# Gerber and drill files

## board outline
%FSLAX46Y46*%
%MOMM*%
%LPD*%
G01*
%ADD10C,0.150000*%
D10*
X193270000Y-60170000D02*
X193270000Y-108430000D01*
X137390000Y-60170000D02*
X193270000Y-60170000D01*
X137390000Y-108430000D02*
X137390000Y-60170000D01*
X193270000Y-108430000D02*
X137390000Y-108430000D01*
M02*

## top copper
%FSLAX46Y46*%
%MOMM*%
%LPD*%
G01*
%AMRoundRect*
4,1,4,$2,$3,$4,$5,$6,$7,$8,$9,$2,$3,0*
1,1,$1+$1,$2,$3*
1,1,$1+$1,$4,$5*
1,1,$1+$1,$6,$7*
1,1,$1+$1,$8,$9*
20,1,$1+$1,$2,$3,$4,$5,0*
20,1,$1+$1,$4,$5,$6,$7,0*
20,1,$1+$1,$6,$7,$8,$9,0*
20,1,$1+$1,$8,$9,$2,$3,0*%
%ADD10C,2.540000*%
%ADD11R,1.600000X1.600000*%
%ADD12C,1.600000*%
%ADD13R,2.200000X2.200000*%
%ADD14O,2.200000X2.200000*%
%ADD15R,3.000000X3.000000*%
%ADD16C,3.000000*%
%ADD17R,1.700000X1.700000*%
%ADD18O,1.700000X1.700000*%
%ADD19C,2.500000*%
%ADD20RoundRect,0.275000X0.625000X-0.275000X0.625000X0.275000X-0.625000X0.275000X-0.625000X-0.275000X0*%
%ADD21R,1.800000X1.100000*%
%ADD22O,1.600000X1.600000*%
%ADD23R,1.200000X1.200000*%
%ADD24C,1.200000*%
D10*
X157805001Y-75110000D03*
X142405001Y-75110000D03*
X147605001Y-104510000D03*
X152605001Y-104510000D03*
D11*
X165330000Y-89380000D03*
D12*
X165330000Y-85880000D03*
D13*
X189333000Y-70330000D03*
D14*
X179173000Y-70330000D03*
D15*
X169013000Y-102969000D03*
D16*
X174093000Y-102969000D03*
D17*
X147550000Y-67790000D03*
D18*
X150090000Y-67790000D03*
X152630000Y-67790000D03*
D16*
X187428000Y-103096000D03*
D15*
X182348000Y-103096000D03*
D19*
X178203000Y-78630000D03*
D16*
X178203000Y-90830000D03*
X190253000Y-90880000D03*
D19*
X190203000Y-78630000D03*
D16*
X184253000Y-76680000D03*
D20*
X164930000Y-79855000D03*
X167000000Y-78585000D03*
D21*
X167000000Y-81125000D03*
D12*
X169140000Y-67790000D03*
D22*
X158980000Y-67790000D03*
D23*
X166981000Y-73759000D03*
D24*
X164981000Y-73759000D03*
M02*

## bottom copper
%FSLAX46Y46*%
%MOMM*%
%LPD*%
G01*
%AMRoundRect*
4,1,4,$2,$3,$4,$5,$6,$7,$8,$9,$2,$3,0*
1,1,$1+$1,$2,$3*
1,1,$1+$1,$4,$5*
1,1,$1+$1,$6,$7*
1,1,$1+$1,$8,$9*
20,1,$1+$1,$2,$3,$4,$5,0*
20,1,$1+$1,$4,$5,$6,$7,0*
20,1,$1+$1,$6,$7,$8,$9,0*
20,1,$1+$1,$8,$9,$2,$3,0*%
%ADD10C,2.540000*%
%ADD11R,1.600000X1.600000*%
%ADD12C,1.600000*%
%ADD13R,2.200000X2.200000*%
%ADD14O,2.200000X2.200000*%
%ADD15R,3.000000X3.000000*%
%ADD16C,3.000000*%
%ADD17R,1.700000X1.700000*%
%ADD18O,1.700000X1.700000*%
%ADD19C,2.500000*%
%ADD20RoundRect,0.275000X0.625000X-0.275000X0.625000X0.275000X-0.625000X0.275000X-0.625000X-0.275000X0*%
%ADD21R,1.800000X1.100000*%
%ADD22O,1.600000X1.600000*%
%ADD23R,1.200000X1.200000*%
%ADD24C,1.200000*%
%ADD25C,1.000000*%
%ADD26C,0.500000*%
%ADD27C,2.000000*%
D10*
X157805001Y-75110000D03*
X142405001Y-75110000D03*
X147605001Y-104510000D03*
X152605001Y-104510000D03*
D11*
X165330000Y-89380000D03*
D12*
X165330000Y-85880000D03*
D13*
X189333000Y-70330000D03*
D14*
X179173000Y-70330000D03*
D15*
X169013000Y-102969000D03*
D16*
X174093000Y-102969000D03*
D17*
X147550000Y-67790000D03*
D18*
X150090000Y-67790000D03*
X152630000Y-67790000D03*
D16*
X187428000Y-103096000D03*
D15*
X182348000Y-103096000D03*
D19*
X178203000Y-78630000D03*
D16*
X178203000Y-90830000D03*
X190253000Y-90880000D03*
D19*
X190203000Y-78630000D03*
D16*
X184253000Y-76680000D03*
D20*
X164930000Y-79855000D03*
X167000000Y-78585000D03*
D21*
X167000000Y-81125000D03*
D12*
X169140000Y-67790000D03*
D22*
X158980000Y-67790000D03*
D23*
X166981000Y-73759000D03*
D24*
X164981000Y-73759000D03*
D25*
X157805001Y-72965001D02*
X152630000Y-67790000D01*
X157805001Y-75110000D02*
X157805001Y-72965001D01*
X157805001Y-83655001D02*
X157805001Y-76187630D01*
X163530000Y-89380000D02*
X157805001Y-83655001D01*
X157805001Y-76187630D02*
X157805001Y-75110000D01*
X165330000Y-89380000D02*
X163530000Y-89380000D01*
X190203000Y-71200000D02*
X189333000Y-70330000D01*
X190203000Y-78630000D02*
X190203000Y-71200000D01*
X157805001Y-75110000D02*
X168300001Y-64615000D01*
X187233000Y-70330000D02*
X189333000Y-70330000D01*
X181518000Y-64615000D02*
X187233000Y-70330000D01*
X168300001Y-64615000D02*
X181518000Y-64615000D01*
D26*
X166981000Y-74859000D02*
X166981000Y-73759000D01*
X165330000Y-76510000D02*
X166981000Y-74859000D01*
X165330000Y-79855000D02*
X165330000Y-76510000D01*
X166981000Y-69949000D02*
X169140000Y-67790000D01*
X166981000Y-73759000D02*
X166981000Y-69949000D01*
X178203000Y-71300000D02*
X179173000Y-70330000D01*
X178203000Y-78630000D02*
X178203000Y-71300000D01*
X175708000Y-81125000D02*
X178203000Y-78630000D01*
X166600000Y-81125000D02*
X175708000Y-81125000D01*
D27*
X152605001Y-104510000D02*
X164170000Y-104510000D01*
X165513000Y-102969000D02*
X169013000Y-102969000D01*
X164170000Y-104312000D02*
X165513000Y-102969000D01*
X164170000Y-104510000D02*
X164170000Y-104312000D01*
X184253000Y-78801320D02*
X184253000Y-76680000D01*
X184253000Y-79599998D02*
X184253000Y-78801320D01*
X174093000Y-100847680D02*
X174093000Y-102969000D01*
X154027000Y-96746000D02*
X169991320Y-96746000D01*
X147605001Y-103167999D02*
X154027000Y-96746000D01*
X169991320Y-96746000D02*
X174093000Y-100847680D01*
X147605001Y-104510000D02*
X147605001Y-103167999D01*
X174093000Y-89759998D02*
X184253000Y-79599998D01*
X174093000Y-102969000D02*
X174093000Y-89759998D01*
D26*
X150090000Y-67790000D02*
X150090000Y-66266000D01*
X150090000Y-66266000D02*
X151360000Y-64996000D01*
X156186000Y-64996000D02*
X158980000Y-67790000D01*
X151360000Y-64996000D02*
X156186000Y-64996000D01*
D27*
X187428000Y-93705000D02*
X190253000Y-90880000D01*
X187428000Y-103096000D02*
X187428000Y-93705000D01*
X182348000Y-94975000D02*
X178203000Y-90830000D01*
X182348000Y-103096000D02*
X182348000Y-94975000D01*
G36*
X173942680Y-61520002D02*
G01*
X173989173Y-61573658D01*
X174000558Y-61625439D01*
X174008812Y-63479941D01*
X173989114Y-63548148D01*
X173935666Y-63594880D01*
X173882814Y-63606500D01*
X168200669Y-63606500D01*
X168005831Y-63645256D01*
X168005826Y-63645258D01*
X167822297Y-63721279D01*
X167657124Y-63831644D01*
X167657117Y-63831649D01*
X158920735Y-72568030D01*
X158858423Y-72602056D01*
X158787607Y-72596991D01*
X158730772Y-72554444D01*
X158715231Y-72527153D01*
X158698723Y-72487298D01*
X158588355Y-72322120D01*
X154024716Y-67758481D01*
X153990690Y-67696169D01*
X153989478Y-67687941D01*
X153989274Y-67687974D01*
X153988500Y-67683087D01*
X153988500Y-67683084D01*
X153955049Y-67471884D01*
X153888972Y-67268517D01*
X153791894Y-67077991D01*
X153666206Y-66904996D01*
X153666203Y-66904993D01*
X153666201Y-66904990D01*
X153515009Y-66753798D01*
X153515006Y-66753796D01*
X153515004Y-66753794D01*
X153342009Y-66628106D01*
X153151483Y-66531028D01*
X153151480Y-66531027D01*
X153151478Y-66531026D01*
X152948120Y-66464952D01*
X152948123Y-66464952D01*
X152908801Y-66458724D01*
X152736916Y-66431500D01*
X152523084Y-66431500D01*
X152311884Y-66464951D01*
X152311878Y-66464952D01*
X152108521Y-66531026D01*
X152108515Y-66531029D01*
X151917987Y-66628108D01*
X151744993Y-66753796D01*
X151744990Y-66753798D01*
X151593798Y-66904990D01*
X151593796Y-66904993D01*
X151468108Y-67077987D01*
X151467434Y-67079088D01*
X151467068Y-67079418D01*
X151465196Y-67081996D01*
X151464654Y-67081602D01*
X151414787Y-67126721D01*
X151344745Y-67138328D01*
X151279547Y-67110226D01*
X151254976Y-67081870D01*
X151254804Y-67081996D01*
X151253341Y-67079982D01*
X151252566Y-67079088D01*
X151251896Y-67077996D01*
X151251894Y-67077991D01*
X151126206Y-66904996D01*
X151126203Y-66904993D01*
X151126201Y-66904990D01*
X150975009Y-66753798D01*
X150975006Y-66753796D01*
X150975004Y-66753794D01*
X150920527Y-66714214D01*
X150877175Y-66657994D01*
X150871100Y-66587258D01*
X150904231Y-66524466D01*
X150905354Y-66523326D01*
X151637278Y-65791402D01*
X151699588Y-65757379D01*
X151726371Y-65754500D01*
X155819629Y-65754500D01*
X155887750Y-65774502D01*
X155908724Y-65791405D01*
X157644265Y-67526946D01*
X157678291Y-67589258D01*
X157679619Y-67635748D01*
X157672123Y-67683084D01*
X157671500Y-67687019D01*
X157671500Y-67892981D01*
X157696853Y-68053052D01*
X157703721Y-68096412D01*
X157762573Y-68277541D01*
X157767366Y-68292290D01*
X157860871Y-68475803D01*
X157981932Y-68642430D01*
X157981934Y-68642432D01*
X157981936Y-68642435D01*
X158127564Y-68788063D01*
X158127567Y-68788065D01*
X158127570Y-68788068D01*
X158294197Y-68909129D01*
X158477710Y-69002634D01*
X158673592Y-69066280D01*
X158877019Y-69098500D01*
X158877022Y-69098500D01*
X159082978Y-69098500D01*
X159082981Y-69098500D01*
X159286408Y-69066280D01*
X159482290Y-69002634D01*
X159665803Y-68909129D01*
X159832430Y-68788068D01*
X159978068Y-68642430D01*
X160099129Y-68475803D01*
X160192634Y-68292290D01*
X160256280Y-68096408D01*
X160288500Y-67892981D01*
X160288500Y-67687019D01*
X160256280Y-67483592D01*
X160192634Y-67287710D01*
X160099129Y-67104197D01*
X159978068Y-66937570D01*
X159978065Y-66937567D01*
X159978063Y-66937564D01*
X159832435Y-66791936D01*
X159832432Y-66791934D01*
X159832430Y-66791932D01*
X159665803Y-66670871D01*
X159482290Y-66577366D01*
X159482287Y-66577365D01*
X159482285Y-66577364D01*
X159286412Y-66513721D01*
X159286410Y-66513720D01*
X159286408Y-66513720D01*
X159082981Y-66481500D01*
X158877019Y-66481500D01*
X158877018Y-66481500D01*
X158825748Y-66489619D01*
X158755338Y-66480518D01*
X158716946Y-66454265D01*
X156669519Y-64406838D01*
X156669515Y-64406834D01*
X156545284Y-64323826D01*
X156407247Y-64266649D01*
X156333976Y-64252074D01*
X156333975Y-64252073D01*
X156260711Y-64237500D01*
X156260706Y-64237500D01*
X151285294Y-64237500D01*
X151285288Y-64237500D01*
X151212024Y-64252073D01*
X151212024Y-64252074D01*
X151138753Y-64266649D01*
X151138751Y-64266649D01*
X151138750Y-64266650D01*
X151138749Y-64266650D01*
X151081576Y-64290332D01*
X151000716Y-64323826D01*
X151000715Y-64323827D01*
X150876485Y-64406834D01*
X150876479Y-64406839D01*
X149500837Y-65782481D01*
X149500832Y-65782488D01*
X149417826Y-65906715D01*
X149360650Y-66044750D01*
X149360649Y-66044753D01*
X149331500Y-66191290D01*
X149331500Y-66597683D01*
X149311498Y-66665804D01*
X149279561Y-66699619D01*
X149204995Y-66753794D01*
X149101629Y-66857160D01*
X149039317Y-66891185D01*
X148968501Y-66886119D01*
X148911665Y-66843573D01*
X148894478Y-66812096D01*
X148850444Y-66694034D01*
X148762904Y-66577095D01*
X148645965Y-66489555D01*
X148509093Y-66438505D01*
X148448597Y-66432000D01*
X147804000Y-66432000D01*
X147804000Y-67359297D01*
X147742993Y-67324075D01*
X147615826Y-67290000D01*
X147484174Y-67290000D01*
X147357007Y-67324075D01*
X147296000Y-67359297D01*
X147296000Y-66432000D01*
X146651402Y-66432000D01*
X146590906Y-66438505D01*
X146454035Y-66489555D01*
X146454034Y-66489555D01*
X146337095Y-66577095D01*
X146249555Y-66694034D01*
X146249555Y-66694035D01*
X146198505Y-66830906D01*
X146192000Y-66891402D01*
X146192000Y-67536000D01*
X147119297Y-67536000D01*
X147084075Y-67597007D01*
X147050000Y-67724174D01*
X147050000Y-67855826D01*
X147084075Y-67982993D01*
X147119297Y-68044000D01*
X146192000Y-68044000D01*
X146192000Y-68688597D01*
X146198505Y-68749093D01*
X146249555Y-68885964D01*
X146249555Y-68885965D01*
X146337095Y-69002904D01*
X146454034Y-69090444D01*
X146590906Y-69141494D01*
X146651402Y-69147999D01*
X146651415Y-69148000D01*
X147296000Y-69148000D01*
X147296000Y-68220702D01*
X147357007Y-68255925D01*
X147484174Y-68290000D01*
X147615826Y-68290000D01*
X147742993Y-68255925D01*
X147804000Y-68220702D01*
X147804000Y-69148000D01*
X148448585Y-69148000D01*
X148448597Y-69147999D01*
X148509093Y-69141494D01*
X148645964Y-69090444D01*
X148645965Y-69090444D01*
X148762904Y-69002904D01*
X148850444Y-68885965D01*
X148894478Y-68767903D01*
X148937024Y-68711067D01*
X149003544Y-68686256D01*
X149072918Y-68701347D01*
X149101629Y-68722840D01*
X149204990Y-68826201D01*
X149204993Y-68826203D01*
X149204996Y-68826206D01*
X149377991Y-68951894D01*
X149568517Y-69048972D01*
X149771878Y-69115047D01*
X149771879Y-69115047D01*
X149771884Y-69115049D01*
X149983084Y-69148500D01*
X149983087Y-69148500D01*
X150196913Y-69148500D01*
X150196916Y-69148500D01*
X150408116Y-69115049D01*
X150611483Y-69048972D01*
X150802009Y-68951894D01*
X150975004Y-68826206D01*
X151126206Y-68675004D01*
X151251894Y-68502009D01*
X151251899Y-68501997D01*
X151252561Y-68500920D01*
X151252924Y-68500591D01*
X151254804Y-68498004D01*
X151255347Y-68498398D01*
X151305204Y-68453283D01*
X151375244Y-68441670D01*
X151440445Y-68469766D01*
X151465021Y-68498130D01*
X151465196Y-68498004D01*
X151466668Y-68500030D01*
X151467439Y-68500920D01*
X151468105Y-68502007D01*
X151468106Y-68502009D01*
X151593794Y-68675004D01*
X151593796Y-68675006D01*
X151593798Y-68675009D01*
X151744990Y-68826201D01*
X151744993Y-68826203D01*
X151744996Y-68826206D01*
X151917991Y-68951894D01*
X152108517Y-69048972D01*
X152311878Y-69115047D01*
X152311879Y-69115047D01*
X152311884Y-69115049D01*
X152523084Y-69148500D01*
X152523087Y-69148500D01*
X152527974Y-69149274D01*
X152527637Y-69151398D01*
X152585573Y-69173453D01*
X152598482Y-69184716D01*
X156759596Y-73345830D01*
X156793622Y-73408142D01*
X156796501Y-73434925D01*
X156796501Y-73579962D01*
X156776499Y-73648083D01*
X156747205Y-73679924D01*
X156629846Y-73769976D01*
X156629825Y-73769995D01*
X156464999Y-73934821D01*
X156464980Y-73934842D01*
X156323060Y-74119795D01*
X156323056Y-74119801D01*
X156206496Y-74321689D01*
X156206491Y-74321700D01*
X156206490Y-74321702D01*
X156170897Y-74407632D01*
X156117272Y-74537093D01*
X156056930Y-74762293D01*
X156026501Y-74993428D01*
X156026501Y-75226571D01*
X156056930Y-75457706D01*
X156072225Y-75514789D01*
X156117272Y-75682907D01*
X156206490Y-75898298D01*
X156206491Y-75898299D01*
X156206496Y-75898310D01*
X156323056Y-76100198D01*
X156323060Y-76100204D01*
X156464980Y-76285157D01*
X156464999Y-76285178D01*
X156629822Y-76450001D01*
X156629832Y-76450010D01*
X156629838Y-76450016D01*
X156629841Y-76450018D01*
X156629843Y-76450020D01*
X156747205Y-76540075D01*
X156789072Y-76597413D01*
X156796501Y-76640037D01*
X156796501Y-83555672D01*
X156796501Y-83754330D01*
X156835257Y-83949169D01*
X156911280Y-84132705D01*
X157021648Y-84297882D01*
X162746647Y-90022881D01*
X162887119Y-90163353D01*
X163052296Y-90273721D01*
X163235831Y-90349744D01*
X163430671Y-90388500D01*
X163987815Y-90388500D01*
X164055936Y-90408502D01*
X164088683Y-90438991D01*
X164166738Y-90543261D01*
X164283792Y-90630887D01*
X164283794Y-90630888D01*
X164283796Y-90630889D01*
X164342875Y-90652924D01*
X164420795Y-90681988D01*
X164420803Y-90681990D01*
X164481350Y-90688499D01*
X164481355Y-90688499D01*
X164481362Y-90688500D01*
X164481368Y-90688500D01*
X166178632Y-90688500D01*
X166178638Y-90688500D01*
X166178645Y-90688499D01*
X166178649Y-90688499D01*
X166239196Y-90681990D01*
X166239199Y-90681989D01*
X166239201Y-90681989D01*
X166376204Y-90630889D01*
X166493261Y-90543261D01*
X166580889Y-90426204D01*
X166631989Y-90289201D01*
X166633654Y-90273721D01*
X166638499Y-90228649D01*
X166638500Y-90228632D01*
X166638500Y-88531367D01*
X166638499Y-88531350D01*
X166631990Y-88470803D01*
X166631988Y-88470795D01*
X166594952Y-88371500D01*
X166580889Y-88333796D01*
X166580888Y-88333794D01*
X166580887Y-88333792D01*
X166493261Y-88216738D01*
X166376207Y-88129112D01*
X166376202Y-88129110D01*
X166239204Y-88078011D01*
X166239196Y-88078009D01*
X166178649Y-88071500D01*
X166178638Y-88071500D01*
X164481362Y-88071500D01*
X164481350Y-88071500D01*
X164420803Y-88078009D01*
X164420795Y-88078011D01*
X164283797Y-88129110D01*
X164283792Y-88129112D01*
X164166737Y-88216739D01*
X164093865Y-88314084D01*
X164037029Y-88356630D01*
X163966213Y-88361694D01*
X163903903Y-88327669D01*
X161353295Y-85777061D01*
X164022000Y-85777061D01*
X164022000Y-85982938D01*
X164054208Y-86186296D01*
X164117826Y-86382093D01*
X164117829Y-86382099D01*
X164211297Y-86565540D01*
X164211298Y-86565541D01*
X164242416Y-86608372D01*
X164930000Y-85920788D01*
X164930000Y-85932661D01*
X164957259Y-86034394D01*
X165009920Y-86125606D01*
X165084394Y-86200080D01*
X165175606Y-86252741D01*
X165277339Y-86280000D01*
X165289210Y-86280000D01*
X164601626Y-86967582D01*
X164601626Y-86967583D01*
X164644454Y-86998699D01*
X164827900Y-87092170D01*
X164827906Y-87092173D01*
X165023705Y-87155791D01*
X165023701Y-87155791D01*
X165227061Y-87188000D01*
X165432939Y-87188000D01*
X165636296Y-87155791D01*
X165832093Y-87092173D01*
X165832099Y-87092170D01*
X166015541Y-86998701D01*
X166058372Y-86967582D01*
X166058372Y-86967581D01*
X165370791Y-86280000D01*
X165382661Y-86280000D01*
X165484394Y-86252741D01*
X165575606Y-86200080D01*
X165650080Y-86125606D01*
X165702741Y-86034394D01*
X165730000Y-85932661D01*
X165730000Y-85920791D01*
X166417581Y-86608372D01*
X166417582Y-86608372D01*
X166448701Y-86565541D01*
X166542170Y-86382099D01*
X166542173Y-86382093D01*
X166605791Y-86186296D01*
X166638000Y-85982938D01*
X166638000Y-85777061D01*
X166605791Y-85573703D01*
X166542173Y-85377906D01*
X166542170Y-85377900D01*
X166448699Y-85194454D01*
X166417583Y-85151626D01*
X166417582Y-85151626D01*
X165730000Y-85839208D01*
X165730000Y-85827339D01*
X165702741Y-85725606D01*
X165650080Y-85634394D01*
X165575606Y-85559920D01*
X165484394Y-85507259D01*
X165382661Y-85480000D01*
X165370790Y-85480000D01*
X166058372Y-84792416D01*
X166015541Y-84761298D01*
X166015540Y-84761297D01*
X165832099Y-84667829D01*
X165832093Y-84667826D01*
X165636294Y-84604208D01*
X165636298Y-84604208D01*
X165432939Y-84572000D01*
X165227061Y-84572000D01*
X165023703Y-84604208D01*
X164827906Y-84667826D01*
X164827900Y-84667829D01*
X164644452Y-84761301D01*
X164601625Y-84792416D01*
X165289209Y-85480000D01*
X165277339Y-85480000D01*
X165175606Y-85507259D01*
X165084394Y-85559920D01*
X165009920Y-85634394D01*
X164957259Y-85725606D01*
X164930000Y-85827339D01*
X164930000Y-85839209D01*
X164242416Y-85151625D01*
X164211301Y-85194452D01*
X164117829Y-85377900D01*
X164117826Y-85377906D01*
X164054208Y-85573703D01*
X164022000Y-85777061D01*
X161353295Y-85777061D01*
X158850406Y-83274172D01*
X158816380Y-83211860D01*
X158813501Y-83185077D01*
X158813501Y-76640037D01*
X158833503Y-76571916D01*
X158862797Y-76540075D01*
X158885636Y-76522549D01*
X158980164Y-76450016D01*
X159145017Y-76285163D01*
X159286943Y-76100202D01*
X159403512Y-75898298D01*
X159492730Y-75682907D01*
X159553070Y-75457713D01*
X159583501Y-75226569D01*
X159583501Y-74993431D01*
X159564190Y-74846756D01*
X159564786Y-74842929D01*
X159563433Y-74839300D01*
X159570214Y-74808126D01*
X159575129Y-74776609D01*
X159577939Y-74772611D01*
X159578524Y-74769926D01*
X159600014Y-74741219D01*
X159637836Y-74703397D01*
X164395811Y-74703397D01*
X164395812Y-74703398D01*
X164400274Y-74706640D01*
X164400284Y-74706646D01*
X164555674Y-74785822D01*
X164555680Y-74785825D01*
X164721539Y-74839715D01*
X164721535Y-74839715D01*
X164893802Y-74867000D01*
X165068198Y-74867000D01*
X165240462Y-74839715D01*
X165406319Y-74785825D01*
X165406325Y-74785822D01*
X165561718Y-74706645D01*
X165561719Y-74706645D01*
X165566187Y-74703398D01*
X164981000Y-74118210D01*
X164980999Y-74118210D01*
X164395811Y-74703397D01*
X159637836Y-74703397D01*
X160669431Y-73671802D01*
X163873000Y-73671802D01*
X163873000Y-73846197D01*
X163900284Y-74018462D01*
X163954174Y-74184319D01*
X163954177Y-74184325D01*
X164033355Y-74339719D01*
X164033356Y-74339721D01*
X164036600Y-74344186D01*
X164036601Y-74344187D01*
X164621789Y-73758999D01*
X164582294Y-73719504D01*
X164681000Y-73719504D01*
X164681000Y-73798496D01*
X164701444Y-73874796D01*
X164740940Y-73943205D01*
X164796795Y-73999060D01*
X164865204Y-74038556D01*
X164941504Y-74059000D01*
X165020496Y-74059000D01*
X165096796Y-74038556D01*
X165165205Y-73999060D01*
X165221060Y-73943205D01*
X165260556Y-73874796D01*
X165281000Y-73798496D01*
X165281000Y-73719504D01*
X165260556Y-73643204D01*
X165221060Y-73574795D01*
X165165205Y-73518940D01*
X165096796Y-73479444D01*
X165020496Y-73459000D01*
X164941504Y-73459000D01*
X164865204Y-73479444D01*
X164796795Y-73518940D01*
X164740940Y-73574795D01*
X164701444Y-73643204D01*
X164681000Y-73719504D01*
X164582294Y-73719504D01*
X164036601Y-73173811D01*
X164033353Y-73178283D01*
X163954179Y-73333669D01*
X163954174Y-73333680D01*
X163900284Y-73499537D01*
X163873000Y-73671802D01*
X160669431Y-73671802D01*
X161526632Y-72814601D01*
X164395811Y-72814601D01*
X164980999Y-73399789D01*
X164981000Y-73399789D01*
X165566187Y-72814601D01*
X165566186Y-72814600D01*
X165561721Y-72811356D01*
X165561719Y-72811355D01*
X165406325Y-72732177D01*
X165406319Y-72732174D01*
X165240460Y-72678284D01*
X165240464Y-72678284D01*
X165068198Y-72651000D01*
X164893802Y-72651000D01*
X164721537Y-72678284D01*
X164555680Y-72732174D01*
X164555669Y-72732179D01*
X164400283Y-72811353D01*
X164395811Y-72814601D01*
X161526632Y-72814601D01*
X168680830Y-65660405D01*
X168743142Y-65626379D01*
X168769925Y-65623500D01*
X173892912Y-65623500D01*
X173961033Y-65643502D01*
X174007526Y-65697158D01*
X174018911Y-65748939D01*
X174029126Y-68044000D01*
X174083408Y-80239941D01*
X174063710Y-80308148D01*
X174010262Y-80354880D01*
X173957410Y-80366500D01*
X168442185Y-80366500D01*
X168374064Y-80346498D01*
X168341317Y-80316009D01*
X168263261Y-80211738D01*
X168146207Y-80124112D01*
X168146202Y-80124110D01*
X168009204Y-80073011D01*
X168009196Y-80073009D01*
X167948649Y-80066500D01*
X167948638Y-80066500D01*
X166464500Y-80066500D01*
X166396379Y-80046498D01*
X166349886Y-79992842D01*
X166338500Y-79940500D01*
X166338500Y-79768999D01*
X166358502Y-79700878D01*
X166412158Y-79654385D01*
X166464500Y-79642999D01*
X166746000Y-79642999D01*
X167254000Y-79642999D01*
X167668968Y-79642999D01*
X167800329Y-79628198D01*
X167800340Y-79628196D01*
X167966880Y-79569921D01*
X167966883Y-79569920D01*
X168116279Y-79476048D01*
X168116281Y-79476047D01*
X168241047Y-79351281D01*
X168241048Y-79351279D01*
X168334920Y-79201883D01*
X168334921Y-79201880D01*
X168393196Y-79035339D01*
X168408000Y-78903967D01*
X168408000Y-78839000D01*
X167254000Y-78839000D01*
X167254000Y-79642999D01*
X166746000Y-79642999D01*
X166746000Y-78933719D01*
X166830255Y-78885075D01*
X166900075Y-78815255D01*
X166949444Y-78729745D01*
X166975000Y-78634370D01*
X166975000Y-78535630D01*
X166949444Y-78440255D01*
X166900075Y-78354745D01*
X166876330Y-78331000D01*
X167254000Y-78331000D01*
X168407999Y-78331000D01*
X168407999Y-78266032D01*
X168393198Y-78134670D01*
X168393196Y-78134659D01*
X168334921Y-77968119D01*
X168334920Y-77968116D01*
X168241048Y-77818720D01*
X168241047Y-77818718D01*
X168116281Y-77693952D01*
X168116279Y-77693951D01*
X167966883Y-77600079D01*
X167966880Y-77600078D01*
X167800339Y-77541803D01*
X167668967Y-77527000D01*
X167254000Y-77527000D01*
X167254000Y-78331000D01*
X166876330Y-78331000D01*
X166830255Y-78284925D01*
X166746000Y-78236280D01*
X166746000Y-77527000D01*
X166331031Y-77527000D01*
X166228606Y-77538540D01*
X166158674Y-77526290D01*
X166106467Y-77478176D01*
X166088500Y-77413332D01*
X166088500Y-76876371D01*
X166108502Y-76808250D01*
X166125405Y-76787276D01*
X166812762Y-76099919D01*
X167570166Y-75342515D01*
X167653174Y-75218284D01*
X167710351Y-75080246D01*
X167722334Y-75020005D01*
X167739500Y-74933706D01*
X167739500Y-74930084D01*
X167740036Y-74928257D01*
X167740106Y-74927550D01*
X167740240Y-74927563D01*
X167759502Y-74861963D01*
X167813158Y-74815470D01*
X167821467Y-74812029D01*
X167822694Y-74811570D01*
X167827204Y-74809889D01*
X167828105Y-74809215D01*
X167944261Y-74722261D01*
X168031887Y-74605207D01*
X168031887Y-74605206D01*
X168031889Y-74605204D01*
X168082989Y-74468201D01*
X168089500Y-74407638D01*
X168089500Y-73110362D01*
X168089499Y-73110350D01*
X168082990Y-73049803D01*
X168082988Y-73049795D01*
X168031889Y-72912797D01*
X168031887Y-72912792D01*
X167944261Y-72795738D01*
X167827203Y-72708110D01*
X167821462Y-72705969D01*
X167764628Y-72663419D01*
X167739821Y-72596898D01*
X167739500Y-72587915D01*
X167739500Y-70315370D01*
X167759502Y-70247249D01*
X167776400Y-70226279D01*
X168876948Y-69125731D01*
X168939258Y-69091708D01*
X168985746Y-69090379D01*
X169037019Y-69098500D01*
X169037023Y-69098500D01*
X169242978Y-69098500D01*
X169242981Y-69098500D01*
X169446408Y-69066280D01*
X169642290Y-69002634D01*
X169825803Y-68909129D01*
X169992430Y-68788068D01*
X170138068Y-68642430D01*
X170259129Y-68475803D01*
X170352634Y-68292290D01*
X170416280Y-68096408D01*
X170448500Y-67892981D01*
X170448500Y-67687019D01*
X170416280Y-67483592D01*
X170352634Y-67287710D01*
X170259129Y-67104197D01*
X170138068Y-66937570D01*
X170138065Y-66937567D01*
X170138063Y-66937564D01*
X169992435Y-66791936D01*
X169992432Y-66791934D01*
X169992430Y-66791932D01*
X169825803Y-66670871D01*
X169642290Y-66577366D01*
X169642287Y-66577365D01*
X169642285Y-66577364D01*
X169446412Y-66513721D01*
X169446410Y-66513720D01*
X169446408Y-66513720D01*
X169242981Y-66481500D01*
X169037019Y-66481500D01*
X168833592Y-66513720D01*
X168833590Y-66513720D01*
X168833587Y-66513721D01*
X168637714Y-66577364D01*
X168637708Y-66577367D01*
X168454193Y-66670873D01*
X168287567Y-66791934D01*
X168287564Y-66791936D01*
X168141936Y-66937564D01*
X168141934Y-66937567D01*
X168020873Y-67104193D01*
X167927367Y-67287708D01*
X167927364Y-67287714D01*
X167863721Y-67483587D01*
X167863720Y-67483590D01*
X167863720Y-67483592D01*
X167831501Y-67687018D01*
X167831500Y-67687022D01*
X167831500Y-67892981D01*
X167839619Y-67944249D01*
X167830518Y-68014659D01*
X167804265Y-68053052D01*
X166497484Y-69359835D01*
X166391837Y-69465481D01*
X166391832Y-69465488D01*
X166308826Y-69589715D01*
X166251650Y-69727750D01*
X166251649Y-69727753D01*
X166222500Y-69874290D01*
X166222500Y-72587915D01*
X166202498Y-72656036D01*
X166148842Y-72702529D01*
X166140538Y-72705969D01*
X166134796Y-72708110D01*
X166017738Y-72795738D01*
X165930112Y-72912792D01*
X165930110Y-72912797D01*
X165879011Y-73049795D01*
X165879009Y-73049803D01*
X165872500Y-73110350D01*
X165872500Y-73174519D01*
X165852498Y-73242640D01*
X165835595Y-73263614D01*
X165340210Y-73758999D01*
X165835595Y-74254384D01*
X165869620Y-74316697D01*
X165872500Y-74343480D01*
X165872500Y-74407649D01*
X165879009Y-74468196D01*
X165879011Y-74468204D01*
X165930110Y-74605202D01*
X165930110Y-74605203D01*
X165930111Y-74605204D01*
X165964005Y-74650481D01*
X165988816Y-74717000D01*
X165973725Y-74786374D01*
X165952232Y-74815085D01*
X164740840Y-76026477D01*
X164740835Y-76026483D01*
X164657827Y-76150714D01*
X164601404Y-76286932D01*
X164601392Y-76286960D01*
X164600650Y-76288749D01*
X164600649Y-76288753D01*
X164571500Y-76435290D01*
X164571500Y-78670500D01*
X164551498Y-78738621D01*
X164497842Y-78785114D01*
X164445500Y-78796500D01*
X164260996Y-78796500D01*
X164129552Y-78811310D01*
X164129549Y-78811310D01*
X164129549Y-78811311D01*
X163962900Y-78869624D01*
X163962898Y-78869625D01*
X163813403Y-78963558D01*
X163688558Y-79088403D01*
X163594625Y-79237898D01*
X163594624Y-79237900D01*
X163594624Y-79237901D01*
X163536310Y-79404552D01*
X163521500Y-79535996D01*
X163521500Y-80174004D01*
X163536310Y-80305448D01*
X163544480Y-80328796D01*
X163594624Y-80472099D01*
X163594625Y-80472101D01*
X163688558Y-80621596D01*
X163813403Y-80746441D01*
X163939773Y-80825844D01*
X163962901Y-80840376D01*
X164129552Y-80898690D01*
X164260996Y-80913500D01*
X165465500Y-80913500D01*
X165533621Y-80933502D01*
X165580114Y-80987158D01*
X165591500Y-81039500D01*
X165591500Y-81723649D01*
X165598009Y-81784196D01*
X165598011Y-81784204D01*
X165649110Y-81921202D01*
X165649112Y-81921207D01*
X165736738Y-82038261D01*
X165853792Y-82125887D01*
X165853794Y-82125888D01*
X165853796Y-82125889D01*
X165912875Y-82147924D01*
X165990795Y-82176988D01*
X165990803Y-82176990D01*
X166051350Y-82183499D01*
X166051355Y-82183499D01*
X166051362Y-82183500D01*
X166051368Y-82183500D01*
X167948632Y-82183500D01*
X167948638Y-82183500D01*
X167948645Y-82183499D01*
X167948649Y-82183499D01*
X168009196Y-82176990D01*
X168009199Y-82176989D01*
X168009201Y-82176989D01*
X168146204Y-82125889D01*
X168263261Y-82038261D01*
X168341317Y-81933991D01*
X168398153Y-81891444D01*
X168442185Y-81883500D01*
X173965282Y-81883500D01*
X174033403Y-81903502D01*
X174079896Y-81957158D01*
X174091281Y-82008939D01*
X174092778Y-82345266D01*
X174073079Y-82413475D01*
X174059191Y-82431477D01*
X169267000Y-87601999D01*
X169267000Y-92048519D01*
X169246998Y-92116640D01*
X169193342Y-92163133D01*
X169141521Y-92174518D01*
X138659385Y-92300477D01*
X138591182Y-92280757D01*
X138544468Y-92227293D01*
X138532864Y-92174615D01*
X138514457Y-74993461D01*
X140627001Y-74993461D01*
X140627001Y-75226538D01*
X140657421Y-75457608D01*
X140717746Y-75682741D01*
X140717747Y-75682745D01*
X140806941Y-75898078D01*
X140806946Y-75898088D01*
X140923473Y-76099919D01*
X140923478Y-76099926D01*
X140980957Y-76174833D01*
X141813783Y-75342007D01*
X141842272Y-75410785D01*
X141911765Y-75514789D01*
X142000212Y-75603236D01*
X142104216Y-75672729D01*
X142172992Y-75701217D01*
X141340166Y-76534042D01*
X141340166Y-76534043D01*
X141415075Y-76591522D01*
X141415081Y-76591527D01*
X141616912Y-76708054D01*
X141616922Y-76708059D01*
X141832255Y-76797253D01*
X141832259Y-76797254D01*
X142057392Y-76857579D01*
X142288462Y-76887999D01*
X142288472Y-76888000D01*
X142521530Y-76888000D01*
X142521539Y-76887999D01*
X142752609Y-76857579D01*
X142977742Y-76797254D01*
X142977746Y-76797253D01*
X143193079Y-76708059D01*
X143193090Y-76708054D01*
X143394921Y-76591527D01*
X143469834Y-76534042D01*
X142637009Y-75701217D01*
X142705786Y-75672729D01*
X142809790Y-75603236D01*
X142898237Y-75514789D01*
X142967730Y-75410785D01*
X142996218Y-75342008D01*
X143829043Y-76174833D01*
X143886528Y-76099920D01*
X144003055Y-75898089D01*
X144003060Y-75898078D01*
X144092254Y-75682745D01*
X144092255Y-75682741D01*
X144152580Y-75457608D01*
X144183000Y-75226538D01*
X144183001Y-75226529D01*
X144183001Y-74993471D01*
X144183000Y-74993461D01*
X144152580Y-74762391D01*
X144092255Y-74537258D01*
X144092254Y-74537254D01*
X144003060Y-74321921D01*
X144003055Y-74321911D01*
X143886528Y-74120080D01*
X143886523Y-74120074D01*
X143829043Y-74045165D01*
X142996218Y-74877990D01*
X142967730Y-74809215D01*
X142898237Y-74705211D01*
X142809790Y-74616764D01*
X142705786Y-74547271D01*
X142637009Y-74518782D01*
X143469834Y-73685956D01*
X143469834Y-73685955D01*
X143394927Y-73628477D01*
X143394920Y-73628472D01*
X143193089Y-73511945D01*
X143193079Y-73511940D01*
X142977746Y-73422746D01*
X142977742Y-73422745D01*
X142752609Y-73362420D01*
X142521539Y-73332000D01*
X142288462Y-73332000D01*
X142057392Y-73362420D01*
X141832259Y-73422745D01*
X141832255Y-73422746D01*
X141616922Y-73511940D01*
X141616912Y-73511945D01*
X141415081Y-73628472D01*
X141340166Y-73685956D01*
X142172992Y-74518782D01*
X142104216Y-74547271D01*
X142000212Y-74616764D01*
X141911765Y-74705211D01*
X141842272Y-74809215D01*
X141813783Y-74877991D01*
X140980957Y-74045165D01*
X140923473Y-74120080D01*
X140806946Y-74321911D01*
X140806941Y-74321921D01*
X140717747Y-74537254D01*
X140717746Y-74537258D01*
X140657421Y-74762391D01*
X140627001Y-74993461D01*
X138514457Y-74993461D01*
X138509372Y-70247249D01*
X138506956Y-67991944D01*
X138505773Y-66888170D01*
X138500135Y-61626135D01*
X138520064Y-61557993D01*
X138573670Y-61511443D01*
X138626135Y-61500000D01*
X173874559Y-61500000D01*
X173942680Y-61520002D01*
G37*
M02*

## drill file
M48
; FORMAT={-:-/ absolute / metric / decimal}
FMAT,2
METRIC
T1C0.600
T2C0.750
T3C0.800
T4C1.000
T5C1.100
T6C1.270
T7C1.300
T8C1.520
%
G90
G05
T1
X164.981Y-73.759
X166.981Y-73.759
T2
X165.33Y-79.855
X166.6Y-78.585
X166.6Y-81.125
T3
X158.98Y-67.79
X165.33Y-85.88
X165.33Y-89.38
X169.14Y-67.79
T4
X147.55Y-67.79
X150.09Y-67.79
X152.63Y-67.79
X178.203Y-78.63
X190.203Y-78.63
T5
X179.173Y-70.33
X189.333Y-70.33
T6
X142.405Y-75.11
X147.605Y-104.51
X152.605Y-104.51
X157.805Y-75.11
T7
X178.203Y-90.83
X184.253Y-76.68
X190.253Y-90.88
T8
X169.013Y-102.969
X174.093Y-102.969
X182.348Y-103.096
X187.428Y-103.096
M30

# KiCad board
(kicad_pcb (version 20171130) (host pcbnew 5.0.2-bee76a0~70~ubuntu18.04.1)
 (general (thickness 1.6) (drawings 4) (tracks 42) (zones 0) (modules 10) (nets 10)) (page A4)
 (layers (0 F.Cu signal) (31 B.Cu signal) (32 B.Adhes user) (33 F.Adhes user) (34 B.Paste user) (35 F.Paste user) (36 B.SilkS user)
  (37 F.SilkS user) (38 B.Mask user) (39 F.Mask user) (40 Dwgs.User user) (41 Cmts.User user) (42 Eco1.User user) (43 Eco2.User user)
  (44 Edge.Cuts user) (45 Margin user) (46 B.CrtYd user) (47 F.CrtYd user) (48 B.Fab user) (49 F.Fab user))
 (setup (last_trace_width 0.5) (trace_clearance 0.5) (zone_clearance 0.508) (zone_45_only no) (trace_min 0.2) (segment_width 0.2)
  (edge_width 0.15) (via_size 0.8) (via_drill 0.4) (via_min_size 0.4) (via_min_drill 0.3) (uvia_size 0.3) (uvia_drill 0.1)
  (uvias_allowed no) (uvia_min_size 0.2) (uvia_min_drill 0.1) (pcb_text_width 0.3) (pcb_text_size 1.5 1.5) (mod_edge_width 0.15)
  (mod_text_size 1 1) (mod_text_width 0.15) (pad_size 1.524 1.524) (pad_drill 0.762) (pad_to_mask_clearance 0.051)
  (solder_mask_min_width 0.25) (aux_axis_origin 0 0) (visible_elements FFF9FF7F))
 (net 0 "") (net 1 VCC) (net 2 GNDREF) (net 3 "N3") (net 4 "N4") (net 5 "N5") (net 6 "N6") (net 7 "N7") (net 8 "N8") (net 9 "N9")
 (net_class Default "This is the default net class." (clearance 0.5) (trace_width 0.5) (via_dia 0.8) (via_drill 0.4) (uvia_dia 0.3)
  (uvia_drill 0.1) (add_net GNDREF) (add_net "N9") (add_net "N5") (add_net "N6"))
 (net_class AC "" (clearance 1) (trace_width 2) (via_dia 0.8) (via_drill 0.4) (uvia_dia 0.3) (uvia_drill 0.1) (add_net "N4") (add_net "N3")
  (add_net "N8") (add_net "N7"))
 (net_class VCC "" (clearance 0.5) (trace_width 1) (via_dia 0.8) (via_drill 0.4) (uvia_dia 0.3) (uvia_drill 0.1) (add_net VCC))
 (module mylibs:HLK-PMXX (layer F.Cu) (at 160.205001 106.91 90)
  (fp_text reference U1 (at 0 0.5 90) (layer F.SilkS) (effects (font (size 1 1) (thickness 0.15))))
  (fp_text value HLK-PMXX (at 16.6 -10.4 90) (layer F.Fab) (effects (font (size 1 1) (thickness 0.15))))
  (pad 4 thru_hole circle (at 31.8 -2.4 90) (size 2.54 2.54) (drill 1.27) (layers *.Cu *.Mask) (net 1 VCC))
  (pad 3 thru_hole circle (at 31.8 -17.8 90) (size 2.54 2.54) (drill 1.27) (layers *.Cu *.Mask) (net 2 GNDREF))
  (pad 1 thru_hole circle (at 2.4 -12.6 90) (size 2.54 2.54) (drill 1.27) (layers *.Cu *.Mask) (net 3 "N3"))
  (pad 2 thru_hole circle (at 2.4 -7.6 90) (size 2.54 2.54) (drill 1.27) (layers *.Cu *.Mask) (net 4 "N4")))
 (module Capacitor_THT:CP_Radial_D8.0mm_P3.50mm (layer F.Cu) (at 165.33 89.38 90)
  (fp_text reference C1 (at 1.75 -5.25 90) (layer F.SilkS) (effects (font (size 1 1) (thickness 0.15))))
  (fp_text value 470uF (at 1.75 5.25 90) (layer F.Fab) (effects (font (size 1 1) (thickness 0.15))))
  (pad 1 thru_hole rect (at 0 0 90) (size 1.6 1.6) (drill 0.8) (layers *.Cu *.Mask) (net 1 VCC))
  (pad 2 thru_hole circle (at 3.5 0 90) (size 1.6 1.6) (drill 0.8) (layers *.Cu *.Mask) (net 2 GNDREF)))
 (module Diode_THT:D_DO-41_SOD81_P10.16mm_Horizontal (layer F.Cu) (at 189.333 70.33 180)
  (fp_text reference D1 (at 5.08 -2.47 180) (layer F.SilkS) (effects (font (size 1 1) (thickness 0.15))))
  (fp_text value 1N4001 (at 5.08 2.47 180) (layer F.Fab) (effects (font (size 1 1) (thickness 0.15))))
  (pad 1 thru_hole rect (at 0 0 180) (size 2.2 2.2) (drill 1.1) (layers *.Cu *.Mask) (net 1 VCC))
  (pad 2 thru_hole oval (at 10.16 0 180) (size 2.2 2.2) (drill 1.1) (layers *.Cu *.Mask) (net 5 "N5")))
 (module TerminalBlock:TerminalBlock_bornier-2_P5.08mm (layer F.Cu) (at 169.013 102.969)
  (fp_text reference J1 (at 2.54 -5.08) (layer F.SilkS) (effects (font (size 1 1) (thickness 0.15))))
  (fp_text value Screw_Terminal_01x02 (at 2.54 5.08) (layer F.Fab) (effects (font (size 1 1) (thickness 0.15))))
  (pad 1 thru_hole rect (at 0 0) (size 3 3) (drill 1.52) (layers *.Cu *.Mask) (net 4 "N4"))
  (pad 2 thru_hole circle (at 5.08 0) (size 3 3) (drill 1.52) (layers *.Cu *.Mask) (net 3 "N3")))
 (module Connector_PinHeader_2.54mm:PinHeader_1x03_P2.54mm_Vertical (layer F.Cu) (at 147.55 67.79 90)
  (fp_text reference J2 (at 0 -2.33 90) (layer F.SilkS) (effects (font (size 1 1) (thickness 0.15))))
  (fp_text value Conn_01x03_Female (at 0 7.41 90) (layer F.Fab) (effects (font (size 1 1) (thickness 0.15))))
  (pad 1 thru_hole rect (at 0 0 90) (size 1.7 1.7) (drill 1) (layers *.Cu *.Mask) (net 2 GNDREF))
  (pad 2 thru_hole oval (at 0 2.54 90) (size 1.7 1.7) (drill 1) (layers *.Cu *.Mask) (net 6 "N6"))
  (pad 3 thru_hole oval (at 0 5.08 90) (size 1.7 1.7) (drill 1) (layers *.Cu *.Mask) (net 1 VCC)))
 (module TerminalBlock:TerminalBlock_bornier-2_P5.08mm (layer F.Cu) (at 182.348 103.096)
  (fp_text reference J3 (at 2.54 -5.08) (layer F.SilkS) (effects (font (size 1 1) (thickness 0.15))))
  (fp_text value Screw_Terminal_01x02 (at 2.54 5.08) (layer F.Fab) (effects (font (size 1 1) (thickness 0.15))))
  (pad 2 thru_hole circle (at 5.08 0) (size 3 3) (drill 1.52) (layers *.Cu *.Mask) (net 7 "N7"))
  (pad 1 thru_hole rect (at 0 0) (size 3 3) (drill 1.52) (layers *.Cu *.Mask) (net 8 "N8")))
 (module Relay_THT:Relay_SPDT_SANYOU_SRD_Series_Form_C (layer F.Cu) (at 184.253 76.68 270)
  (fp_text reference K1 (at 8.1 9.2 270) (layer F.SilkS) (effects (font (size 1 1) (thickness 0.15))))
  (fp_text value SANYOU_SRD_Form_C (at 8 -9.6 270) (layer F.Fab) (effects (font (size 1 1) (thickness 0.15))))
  (pad 2 thru_hole circle (at 1.95 6.05) (size 2.5 2.5) (drill 1) (layers *.Cu *.Mask) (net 5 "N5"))
  (pad 3 thru_hole circle (at 14.15 6.05) (size 3 3) (drill 1.3) (layers *.Cu *.Mask) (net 8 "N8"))
  (pad 4 thru_hole circle (at 14.2 -6) (size 3 3) (drill 1.3) (layers *.Cu *.Mask) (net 7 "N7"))
  (pad 5 thru_hole circle (at 1.95 -5.95) (size 2.5 2.5) (drill 1) (layers *.Cu *.Mask) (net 1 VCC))
  (pad 1 thru_hole circle (at 0 0) (size 3 3) (drill 1.3) (layers *.Cu *.Mask) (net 3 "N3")))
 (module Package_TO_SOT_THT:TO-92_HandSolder (layer F.Cu) (at 166.6 81.125 90)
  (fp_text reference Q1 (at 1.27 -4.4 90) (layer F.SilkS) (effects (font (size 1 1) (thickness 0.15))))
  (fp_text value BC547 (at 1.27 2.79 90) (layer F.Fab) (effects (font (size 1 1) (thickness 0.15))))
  (pad 2 thru_hole roundrect (at 1.27 -1.27 90) (size 1.1 1.8) (drill 0.75 (offset 0 -0.4)) (layers *.Cu *.Mask) (roundrect_rratio 0.25)
   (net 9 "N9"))
  (pad 3 thru_hole roundrect (at 2.54 0 90) (size 1.1 1.8) (drill 0.75 (offset 0 0.4)) (layers *.Cu *.Mask) (roundrect_rratio 0.25)
   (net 2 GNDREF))
  (pad 1 thru_hole rect (at 0 0 90) (size 1.1 1.8) (drill 0.75 (offset 0 0.4)) (layers *.Cu *.Mask) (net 5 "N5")))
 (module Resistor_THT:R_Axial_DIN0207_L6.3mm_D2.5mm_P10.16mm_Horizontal (layer F.Cu) (at 169.14 67.79 180)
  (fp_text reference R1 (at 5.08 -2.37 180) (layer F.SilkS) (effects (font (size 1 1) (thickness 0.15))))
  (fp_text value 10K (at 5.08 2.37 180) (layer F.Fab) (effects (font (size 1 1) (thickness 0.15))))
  (pad 1 thru_hole circle (at 0 0 180) (size 1.6 1.6) (drill 0.8) (layers *.Cu *.Mask) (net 9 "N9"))
  (pad 2 thru_hole oval (at 10.16 0 180) (size 1.6 1.6) (drill 0.8) (layers *.Cu *.Mask) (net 6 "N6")))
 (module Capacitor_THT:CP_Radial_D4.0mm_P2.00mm (layer F.Cu) (at 166.981 73.759 180)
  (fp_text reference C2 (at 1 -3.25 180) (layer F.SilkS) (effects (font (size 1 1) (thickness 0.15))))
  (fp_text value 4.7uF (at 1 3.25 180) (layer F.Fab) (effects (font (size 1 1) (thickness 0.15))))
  (pad 1 thru_hole rect (at 0 0 180) (size 1.2 1.2) (drill 0.6) (layers *.Cu *.Mask) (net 9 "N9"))
  (pad 2 thru_hole circle (at 2 0 180) (size 1.2 1.2) (drill 0.6) (layers *.Cu *.Mask) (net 2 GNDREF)))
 (gr_line (start 193.27 60.17) (end 193.27 108.43) (layer Edge.Cuts) (width 0.15))
 (gr_line (start 137.39 60.17) (end 193.27 60.17) (layer Edge.Cuts) (width 0.15))
 (gr_line (start 137.39 108.43) (end 137.39 60.17) (layer Edge.Cuts) (width 0.15))
 (gr_line (start 193.27 108.43) (end 137.39 108.43) (layer Edge.Cuts) (width 0.15))
 (segment (start 157.805001 72.965001) (end 152.63 67.79) (width 1) (layer B.Cu) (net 1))
 (segment (start 157.805001 75.11) (end 157.805001 72.965001) (width 1) (layer B.Cu) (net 1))
 (segment (start 157.805001 83.655001) (end 157.805001 76.18763) (width 1) (layer B.Cu) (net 1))
 (segment (start 163.53 89.38) (end 157.805001 83.655001) (width 1) (layer B.Cu) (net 1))
 (segment (start 157.805001 76.18763) (end 157.805001 75.11) (width 1) (layer B.Cu) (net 1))
 (segment (start 165.33 89.38) (end 163.53 89.38) (width 1) (layer B.Cu) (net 1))
 (segment (start 190.203 71.2) (end 189.333 70.33) (width 1) (layer B.Cu) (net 1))
 (segment (start 190.203 78.63) (end 190.203 71.2) (width 1) (layer B.Cu) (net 1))
 (segment (start 157.805001 75.11) (end 168.300001 64.615) (width 1) (layer B.Cu) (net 1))
 (segment (start 187.233 70.33) (end 189.333 70.33) (width 1) (layer B.Cu) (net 1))
 (segment (start 181.518 64.615) (end 187.233 70.33) (width 1) (layer B.Cu) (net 1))
 (segment (start 168.300001 64.615) (end 181.518 64.615) (width 1) (layer B.Cu) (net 1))
 (segment (start 166.981 74.859) (end 166.981 73.759) (width 0.5) (layer B.Cu) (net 9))
 (segment (start 165.33 76.51) (end 166.981 74.859) (width 0.5) (layer B.Cu) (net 9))
 (segment (start 165.33 79.855) (end 165.33 76.51) (width 0.5) (layer B.Cu) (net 9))
 (segment (start 166.981 69.949) (end 169.14 67.79) (width 0.5) (layer B.Cu) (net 9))
 (segment (start 166.981 73.759) (end 166.981 69.949) (width 0.5) (layer B.Cu) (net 9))
 (segment (start 178.203 71.3) (end 179.173 70.33) (width 0.5) (layer B.Cu) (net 5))
 (segment (start 178.203 78.63) (end 178.203 71.3) (width 0.5) (layer B.Cu) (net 5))
 (segment (start 175.708 81.125) (end 178.203 78.63) (width 0.5) (layer B.Cu) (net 5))
 (segment (start 166.6 81.125) (end 175.708 81.125) (width 0.5) (layer B.Cu) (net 5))
 (segment (start 152.605001 104.51) (end 164.17 104.51) (width 2) (layer B.Cu) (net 4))
 (segment (start 165.513 102.969) (end 169.013 102.969) (width 2) (layer B.Cu) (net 4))
 (segment (start 164.17 104.312) (end 165.513 102.969) (width 2) (layer B.Cu) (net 4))
 (segment (start 164.17 104.51) (end 164.17 104.312) (width 2) (layer B.Cu) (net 4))
 (segment (start 184.253 78.80132) (end 184.253 76.68) (width 2) (layer B.Cu) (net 3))
 (segment (start 184.253 79.599998) (end 184.253 78.80132) (width 2) (layer B.Cu) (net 3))
 (segment (start 174.093 100.84768) (end 174.093 102.969) (width 2) (layer B.Cu) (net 3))
 (segment (start 154.027 96.746) (end 169.99132 96.746) (width 2) (layer B.Cu) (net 3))
 (segment (start 147.605001 103.167999) (end 154.027 96.746) (width 2) (layer B.Cu) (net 3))
 (segment (start 169.99132 96.746) (end 174.093 100.84768) (width 2) (layer B.Cu) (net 3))
 (segment (start 147.605001 104.51) (end 147.605001 103.167999) (width 2) (layer B.Cu) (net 3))
 (segment (start 174.093 89.759998) (end 184.253 79.599998) (width 2) (layer B.Cu) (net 3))
 (segment (start 174.093 102.969) (end 174.093 89.759998) (width 2) (layer B.Cu) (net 3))
 (segment (start 150.09 67.79) (end 150.09 66.266) (width 0.5) (layer B.Cu) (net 6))
 (segment (start 150.09 66.266) (end 151.36 64.996) (width 0.5) (layer B.Cu) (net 6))
 (segment (start 156.186 64.996) (end 158.98 67.79) (width 0.5) (layer B.Cu) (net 6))
 (segment (start 151.36 64.996) (end 156.186 64.996) (width 0.5) (layer B.Cu) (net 6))
 (segment (start 187.428 93.705) (end 190.253 90.88) (width 2) (layer B.Cu) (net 7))
 (segment (start 187.428 103.096) (end 187.428 93.705) (width 2) (layer B.Cu) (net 7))
 (segment (start 182.348 94.975) (end 178.203 90.83) (width 2) (layer B.Cu) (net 8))
 (segment (start 182.348 103.096) (end 182.348 94.975) (width 2) (layer B.Cu) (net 8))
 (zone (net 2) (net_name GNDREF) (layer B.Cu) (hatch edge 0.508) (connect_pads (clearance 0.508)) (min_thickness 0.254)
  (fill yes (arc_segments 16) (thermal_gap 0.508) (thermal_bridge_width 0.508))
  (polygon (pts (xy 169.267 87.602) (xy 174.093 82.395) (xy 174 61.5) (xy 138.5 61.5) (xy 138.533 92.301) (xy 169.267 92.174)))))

